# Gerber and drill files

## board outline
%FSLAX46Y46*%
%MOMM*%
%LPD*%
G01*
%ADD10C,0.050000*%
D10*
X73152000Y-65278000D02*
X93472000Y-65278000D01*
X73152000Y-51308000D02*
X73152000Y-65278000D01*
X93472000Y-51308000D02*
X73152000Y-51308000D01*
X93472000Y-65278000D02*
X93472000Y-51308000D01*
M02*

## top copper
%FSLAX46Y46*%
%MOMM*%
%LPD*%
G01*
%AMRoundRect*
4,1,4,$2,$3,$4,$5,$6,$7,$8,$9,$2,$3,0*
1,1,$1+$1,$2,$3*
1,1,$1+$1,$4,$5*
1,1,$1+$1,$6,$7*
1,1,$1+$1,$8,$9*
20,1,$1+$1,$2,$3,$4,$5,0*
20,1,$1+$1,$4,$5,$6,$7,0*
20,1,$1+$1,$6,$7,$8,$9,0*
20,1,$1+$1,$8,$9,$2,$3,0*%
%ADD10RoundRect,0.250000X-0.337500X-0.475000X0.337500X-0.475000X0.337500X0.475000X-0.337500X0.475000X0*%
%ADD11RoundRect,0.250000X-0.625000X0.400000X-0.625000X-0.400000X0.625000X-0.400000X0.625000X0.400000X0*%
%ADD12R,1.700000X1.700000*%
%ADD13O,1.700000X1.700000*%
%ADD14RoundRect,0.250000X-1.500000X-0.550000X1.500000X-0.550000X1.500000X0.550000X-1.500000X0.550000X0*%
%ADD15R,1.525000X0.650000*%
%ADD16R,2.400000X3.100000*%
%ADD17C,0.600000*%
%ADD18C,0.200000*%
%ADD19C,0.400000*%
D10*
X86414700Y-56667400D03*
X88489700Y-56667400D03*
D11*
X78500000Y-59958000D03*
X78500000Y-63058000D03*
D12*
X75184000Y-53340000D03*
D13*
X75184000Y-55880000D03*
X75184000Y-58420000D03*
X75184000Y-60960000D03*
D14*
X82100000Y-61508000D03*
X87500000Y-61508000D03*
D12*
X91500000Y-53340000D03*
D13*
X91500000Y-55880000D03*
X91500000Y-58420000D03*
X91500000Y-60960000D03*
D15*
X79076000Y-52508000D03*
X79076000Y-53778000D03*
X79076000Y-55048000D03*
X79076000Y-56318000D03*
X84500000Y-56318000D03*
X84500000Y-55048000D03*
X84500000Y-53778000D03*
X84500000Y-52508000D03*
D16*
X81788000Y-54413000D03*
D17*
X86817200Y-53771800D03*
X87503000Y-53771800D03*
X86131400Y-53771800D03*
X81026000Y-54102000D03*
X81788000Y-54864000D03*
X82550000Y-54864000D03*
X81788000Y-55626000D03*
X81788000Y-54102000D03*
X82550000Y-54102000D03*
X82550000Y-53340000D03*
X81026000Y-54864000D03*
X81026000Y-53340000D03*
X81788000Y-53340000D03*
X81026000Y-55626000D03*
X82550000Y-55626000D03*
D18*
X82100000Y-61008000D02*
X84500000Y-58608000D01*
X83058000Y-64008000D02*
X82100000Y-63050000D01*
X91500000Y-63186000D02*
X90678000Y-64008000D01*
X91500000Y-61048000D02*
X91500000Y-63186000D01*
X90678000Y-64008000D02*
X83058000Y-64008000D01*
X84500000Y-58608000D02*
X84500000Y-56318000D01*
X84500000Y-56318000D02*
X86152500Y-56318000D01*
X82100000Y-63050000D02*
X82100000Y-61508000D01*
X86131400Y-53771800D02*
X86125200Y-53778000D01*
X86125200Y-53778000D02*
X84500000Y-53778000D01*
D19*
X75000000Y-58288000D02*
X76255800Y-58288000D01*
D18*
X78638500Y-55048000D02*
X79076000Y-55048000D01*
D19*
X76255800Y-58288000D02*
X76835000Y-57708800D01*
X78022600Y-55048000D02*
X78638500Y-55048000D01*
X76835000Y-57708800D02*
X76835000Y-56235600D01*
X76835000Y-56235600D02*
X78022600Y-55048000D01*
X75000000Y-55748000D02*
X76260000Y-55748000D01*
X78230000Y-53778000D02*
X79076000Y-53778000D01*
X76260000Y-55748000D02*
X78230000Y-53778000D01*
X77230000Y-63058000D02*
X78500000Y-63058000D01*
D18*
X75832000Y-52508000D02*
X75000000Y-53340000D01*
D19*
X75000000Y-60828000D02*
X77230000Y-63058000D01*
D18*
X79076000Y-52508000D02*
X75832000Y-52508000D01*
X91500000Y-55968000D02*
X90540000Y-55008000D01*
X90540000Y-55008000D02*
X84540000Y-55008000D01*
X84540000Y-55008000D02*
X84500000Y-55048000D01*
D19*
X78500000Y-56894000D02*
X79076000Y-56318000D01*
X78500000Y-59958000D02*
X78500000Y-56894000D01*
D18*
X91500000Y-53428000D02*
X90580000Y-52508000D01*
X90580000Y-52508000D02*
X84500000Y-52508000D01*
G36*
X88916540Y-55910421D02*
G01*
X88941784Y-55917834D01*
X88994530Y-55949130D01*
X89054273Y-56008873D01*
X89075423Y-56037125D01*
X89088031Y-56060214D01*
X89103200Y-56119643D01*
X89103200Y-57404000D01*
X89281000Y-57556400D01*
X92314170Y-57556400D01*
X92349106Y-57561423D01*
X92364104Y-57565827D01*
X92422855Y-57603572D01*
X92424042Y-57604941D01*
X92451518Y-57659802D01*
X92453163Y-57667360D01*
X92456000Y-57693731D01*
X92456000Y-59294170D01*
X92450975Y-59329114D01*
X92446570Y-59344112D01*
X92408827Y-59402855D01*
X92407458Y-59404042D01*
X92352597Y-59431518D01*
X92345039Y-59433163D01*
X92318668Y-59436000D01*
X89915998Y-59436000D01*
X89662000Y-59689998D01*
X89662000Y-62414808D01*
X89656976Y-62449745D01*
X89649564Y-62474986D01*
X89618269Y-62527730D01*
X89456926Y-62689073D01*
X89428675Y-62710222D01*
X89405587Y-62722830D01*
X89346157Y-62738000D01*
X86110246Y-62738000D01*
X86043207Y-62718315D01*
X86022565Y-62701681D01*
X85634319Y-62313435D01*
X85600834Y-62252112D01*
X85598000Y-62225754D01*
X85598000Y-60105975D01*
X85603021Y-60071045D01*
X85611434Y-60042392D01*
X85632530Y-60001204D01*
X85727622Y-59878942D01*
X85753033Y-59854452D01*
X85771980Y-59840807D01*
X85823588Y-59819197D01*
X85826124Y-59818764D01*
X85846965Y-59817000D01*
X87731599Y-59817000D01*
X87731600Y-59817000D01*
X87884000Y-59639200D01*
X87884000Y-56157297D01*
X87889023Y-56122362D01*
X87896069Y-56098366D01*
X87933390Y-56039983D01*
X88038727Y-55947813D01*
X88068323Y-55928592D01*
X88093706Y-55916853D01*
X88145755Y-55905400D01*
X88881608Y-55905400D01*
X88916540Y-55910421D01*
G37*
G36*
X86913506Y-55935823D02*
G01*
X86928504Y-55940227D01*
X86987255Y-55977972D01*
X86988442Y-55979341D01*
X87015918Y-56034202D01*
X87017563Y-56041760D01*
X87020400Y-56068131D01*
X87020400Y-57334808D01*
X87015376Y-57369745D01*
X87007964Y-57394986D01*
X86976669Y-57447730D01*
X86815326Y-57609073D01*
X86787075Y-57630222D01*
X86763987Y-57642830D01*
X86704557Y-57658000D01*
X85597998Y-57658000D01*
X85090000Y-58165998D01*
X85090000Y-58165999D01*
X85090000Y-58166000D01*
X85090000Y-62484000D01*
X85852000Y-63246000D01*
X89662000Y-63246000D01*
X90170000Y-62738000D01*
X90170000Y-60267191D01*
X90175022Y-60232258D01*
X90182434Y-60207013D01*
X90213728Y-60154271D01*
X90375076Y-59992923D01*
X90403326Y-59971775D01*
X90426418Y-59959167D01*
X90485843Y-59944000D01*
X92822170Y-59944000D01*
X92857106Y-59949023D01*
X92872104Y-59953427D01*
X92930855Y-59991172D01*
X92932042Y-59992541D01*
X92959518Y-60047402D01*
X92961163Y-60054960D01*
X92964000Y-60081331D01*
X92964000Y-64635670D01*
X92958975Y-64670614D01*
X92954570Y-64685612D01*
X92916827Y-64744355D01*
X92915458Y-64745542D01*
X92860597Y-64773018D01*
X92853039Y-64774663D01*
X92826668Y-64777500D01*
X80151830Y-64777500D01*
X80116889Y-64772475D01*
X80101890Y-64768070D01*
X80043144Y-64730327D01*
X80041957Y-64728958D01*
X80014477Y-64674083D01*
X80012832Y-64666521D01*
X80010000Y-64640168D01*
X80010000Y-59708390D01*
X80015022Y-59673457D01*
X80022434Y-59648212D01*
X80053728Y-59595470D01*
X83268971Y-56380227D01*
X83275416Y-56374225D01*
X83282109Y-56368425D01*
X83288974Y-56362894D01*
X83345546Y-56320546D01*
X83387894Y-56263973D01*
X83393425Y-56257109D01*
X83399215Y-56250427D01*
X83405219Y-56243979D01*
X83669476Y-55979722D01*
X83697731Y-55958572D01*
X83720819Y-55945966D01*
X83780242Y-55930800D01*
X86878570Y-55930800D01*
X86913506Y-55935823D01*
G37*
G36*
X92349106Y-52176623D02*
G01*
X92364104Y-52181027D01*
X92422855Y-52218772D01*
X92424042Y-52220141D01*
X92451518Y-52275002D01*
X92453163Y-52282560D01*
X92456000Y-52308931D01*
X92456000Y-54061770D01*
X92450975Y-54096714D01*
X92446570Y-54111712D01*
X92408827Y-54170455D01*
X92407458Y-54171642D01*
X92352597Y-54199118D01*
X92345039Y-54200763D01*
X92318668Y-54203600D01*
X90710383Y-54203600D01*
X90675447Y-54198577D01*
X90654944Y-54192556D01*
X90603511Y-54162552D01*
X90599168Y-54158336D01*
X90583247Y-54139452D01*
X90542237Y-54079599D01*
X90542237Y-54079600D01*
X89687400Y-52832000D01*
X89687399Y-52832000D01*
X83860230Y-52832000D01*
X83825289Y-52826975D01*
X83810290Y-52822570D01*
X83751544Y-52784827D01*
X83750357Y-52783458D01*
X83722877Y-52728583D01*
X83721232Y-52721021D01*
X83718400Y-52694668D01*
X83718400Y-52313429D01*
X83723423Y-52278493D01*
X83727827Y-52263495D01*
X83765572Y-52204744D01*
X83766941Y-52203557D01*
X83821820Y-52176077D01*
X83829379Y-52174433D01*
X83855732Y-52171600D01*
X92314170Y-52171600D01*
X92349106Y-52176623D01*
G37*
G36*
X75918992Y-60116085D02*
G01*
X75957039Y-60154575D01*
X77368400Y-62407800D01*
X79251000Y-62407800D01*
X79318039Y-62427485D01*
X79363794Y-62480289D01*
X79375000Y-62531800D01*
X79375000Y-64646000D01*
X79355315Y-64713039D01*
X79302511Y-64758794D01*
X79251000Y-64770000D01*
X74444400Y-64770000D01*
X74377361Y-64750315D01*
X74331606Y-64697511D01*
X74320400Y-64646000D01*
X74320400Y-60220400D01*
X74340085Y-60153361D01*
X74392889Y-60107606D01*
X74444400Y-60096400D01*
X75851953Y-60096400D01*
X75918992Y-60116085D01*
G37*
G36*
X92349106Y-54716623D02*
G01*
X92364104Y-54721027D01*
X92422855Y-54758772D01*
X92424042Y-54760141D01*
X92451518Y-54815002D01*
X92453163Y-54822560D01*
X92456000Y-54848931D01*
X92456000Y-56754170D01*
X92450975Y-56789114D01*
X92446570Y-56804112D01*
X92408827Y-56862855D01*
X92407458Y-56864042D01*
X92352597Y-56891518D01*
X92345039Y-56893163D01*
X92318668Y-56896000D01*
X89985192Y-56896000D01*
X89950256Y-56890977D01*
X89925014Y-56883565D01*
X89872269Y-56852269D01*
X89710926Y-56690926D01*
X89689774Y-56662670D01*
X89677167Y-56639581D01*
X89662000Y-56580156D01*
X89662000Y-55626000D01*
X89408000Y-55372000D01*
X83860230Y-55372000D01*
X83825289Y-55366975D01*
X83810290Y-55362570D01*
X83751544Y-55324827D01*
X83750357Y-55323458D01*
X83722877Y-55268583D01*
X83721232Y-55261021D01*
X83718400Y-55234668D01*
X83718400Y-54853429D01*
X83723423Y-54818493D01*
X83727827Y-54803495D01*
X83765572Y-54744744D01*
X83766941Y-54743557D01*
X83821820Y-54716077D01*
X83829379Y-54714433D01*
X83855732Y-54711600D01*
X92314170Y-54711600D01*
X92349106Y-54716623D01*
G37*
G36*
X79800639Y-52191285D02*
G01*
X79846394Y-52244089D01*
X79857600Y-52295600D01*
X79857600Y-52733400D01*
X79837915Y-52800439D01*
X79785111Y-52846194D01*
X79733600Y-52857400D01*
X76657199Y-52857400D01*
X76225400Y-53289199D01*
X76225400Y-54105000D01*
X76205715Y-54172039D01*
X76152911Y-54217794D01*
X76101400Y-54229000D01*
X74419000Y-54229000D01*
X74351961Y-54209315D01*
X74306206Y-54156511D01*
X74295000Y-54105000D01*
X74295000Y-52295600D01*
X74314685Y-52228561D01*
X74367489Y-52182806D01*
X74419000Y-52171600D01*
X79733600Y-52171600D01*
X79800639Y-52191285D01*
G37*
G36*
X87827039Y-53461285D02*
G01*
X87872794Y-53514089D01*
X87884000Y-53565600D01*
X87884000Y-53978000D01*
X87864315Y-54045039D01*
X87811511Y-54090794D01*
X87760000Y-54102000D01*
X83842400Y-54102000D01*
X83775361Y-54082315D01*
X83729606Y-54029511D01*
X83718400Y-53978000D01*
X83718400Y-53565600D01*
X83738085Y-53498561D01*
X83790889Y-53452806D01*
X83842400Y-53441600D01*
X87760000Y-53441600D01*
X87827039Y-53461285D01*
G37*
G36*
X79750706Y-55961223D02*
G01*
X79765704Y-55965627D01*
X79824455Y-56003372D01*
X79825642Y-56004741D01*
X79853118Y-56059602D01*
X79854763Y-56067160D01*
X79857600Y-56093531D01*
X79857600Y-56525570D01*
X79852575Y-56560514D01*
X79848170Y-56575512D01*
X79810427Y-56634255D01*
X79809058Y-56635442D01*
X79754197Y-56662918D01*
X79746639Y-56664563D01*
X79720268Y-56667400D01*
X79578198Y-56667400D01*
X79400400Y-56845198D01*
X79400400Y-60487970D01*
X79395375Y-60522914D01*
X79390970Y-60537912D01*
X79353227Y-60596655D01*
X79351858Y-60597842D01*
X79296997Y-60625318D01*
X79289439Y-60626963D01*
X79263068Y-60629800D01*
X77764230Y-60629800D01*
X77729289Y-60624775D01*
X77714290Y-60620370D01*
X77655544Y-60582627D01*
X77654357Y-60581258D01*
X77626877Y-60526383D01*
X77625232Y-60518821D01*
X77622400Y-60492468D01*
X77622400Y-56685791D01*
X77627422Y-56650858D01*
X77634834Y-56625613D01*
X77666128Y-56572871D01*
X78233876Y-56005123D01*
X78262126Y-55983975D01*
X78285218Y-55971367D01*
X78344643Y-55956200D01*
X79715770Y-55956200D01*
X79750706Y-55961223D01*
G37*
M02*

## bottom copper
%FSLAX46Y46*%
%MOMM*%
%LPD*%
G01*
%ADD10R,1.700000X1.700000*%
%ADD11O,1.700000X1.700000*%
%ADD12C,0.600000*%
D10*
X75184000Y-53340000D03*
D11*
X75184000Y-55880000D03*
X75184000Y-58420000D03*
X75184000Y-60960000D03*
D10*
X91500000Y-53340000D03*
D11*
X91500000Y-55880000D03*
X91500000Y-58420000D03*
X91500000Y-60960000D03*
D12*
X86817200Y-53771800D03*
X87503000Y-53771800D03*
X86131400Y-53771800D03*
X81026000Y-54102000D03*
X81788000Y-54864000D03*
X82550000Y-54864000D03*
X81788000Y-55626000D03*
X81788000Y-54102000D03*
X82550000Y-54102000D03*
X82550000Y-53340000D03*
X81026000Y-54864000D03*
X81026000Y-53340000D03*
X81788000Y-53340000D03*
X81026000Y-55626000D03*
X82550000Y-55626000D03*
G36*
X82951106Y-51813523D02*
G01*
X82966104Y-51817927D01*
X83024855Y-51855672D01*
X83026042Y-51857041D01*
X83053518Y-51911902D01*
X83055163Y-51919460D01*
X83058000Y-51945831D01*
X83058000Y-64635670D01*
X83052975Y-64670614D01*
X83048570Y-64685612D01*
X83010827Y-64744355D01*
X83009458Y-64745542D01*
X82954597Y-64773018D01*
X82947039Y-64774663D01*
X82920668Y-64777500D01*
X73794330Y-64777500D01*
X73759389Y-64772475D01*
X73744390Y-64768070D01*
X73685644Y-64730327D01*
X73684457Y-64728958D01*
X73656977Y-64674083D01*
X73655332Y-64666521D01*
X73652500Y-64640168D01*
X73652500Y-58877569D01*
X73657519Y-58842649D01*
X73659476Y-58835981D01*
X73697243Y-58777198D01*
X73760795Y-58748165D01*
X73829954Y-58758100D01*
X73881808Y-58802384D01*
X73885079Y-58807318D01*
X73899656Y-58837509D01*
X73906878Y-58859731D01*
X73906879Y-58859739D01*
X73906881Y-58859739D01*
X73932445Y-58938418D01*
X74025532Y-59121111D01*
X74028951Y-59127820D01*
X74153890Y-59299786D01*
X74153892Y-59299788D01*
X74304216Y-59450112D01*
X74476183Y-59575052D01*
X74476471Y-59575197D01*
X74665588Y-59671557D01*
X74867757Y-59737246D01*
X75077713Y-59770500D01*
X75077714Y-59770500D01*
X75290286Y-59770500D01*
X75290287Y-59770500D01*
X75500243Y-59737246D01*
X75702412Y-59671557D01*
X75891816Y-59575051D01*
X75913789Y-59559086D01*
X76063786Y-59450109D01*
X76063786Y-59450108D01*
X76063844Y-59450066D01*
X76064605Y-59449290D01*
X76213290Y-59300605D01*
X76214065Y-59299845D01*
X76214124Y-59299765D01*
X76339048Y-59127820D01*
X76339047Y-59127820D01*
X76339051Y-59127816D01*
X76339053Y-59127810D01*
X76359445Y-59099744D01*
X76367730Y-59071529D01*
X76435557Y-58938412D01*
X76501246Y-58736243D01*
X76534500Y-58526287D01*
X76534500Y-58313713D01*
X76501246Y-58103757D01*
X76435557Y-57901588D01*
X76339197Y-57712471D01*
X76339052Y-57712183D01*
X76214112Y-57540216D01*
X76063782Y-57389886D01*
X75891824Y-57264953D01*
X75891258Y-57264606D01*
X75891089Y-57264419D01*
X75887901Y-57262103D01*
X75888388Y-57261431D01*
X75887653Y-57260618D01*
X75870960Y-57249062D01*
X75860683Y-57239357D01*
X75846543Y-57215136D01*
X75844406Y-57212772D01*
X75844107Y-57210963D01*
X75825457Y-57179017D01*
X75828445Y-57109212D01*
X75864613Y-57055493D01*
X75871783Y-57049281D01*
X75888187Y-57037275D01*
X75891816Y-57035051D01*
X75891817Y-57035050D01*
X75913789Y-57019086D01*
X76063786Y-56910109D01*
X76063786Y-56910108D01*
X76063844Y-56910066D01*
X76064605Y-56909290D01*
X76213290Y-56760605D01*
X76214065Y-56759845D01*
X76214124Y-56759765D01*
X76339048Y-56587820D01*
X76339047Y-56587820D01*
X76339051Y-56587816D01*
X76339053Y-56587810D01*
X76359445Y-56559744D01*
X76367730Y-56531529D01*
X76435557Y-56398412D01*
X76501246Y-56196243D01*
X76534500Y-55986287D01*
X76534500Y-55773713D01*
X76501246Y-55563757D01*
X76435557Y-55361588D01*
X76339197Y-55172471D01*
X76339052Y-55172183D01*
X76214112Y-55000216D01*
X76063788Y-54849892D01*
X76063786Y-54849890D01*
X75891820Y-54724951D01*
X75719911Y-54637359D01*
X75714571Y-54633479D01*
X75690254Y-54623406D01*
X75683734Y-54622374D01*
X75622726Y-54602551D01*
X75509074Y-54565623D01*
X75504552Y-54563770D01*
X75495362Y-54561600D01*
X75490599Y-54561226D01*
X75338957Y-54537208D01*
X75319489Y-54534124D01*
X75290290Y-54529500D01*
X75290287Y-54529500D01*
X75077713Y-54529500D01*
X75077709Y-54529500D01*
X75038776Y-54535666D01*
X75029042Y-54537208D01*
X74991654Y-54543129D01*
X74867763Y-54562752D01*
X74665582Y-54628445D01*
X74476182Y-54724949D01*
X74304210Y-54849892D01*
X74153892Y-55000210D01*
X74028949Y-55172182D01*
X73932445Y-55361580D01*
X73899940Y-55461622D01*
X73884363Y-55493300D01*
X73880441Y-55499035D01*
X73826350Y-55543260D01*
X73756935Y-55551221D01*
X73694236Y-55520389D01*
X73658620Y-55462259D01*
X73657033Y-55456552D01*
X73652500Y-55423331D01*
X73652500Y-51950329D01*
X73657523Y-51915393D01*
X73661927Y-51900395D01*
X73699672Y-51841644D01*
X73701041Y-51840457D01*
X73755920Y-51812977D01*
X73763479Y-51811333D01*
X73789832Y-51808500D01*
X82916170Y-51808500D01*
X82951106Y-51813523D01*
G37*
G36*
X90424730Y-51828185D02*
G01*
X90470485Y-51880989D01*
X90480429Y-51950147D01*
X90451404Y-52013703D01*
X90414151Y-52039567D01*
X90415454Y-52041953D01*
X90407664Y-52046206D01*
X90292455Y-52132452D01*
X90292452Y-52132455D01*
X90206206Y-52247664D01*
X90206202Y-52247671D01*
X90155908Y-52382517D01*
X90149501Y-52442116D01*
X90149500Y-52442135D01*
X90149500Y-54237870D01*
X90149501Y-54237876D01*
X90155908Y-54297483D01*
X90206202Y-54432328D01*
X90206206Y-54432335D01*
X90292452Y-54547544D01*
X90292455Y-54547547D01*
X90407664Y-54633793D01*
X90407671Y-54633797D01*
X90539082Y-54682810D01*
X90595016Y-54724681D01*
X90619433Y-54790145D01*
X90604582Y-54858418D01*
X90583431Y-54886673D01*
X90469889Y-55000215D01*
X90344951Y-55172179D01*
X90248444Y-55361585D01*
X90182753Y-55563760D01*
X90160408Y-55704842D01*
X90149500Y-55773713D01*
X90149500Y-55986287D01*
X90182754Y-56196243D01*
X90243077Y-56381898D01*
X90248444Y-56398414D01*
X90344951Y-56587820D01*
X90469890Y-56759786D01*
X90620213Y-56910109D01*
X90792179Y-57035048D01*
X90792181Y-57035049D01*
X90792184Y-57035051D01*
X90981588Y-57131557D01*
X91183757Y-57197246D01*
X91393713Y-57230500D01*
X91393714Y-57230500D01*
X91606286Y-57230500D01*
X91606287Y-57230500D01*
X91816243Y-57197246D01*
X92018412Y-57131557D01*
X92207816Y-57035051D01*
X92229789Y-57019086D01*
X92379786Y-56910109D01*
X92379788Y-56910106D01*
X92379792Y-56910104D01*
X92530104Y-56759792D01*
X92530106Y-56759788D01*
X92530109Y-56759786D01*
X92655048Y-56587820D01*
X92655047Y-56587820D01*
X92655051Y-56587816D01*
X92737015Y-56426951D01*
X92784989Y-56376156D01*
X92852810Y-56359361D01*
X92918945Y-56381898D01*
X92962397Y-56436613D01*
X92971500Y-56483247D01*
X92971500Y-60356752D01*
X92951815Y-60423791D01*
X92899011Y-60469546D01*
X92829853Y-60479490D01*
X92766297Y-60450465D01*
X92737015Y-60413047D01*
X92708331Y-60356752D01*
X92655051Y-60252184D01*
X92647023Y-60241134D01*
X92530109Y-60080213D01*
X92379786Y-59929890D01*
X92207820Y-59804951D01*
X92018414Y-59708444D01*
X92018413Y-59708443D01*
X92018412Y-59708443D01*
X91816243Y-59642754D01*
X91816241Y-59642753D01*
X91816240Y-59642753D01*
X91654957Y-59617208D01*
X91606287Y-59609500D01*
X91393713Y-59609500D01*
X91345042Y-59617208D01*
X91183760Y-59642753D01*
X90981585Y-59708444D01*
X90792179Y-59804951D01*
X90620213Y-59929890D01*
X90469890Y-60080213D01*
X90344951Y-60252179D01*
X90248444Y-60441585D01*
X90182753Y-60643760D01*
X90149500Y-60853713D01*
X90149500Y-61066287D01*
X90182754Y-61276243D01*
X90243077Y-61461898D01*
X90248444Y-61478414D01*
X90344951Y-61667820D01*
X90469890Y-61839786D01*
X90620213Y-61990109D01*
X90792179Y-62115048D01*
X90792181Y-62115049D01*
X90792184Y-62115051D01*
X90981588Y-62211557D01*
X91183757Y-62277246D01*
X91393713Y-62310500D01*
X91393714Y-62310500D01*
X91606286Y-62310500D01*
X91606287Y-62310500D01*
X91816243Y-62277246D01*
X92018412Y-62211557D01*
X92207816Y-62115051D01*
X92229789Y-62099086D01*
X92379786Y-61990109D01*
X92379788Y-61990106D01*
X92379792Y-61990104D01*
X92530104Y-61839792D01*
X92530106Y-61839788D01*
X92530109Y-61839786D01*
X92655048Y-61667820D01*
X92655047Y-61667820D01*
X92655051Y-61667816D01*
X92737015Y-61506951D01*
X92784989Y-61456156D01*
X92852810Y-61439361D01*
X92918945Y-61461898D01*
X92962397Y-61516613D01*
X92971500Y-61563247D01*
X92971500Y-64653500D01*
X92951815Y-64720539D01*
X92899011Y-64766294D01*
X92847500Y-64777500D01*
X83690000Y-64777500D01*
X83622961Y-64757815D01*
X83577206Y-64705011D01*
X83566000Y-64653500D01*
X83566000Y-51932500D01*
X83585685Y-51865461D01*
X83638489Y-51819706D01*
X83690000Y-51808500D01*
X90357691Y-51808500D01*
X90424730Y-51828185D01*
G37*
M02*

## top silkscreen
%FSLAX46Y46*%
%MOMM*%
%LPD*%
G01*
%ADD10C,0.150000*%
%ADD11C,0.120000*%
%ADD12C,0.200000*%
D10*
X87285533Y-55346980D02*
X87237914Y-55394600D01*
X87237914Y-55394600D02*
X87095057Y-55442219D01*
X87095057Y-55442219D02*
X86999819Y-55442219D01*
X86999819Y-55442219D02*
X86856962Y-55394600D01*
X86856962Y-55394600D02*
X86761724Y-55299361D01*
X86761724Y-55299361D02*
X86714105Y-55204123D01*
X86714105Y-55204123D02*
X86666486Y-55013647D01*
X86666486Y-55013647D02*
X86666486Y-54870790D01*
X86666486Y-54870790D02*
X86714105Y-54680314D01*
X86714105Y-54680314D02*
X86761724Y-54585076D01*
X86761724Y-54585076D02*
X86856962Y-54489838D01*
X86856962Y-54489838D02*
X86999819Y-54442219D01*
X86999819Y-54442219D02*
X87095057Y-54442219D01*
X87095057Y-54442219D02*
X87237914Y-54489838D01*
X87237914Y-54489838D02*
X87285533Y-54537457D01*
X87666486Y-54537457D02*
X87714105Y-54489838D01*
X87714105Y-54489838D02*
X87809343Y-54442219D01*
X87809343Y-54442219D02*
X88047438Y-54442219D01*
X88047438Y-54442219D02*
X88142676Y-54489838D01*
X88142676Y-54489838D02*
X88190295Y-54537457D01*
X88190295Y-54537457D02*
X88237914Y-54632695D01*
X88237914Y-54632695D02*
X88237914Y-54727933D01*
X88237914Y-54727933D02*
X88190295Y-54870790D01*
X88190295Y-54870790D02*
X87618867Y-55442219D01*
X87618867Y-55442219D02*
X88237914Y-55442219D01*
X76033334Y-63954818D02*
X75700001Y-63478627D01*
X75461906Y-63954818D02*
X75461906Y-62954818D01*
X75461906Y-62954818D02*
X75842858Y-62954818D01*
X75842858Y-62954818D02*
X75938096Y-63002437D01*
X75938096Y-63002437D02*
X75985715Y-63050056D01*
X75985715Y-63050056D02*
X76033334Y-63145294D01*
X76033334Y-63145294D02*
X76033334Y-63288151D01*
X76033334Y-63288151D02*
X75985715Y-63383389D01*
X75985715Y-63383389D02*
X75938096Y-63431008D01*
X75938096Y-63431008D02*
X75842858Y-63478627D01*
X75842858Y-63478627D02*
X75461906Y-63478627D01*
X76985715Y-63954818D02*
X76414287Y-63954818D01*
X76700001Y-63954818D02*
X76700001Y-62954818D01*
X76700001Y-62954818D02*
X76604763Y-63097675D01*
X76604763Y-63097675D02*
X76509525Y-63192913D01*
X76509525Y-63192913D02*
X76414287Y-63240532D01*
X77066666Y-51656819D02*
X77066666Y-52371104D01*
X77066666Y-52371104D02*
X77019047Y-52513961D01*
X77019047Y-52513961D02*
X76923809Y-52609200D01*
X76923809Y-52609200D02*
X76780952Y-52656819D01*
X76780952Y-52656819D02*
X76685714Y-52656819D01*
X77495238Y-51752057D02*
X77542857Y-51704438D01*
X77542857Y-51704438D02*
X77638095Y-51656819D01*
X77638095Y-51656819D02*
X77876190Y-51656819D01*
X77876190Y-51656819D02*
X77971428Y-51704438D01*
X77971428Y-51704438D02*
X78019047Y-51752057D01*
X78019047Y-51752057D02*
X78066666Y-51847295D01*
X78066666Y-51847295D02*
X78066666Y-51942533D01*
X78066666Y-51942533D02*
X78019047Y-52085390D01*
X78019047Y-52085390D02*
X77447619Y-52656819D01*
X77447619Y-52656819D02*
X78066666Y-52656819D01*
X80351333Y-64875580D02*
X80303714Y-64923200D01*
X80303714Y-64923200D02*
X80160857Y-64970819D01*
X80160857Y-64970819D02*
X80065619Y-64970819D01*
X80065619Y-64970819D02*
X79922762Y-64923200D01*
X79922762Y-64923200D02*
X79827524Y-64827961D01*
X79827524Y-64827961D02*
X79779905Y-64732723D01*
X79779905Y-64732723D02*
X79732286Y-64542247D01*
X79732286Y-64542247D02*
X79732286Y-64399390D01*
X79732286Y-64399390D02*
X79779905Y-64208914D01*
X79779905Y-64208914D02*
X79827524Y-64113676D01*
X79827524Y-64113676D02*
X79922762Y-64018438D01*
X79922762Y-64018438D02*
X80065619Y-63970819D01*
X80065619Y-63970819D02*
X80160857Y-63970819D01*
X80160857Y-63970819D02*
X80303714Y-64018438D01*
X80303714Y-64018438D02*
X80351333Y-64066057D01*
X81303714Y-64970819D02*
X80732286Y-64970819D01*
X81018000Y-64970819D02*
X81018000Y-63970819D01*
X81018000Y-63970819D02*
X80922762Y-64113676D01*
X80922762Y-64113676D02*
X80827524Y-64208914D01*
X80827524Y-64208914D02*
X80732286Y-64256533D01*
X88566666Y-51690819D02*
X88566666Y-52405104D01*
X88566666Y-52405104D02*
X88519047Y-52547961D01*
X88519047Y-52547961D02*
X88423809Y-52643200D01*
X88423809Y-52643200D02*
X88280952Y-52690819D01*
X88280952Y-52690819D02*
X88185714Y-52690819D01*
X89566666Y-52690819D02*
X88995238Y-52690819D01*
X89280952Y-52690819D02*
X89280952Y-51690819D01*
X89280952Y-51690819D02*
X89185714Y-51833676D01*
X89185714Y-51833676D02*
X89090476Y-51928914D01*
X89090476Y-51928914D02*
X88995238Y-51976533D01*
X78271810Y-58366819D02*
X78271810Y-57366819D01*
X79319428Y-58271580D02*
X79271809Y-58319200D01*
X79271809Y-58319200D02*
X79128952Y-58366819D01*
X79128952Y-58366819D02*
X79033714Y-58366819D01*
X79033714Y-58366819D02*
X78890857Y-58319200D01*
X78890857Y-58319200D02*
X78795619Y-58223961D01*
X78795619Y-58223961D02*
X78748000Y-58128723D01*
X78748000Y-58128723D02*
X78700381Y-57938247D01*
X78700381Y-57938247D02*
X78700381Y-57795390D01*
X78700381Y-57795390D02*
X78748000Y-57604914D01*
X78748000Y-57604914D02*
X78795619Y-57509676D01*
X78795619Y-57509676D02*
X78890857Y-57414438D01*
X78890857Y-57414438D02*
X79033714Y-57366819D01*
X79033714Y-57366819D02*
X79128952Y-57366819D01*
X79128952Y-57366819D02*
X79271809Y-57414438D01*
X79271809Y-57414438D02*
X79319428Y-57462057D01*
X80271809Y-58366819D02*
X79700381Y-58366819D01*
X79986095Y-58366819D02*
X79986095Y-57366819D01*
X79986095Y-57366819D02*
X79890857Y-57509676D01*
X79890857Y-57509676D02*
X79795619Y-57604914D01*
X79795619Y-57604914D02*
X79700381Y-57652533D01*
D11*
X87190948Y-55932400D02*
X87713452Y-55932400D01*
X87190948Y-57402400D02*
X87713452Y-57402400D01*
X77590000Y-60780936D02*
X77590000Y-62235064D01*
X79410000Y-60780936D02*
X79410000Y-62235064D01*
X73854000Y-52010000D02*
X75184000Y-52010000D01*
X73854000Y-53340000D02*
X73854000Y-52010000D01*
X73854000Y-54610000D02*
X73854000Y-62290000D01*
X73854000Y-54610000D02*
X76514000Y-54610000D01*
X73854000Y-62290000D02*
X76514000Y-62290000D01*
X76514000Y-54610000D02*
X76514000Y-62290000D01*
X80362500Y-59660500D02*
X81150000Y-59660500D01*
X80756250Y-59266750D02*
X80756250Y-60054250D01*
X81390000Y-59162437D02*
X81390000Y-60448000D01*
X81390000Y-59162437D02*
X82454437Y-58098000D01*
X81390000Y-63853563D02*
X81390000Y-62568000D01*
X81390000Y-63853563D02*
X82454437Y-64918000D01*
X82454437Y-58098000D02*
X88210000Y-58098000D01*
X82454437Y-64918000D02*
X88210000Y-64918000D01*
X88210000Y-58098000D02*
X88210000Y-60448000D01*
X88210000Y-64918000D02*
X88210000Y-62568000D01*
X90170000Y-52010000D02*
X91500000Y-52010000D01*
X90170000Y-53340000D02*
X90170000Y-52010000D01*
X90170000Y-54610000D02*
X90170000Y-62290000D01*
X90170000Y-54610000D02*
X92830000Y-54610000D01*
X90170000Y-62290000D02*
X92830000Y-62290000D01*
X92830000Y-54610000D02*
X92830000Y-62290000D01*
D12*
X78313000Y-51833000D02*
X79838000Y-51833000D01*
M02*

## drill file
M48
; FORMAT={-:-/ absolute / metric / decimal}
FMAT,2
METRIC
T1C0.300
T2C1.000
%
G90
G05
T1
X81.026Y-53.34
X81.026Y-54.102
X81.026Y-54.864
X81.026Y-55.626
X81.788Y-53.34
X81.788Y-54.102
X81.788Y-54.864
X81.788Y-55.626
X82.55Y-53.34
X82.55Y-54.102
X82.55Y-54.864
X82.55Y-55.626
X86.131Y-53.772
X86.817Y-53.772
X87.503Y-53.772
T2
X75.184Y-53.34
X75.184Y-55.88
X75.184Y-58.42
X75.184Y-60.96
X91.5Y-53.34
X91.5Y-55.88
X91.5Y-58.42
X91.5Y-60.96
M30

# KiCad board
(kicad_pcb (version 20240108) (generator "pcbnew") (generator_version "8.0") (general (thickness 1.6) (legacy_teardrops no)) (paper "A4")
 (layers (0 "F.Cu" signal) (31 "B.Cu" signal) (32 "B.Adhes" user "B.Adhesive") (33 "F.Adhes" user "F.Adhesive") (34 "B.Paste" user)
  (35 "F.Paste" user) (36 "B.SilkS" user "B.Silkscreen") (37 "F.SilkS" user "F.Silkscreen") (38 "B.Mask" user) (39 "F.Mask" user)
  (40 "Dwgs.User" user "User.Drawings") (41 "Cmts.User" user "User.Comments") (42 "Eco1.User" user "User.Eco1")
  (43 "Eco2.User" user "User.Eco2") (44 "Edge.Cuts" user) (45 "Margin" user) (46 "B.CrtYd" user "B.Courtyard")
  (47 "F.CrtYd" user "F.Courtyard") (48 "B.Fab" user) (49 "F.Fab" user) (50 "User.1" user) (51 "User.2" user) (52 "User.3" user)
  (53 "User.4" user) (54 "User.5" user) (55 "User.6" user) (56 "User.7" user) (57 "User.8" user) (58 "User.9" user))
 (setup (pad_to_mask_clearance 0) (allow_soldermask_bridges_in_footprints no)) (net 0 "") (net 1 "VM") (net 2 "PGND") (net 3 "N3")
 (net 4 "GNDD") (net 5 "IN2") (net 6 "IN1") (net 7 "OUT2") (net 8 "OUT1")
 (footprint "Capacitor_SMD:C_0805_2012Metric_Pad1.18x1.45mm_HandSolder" (layer "F.Cu") (at 87.4522 56.6674)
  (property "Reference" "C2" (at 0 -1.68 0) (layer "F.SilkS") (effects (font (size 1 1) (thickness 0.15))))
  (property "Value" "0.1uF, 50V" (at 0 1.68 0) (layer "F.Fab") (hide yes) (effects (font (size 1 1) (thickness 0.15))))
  (fp_line (start -0.261252 -0.735) (end 0.261252 -0.735) (stroke (width 0.12) (type solid)) (layer "F.SilkS"))
  (fp_line (start -0.261252 0.735) (end 0.261252 0.735) (stroke (width 0.12) (type solid)) (layer "F.SilkS"))
  (pad "1" smd roundrect (at -1.0375 0) (size 1.175 1.45) (layers "F.Cu" "F.Paste" "F.Mask") (roundrect_rratio 0.212766) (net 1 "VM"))
  (pad "2" smd roundrect (at 1.0375 0) (size 1.175 1.45) (layers "F.Cu" "F.Paste" "F.Mask") (roundrect_rratio 0.212766) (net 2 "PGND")))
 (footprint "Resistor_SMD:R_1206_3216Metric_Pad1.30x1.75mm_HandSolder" (layer "F.Cu") (at 78.5 61.508 -90)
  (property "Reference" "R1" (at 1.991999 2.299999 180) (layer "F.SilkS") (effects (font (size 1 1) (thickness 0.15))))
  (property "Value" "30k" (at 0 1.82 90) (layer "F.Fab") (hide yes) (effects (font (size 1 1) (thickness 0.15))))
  (fp_line (start -0.727064 0.91) (end 0.727064 0.91) (stroke (width 0.12) (type solid)) (layer "F.SilkS"))
  (fp_line (start -0.727064 -0.91) (end 0.727064 -0.91) (stroke (width 0.12) (type solid)) (layer "F.SilkS"))
  (pad "1" smd roundrect (at -1.55 0 270) (size 1.3 1.75) (layers "F.Cu" "F.Paste" "F.Mask") (roundrect_rratio 0.192308) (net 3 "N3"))
  (pad "2" smd roundrect (at 1.55 0 270) (size 1.3 1.75) (layers "F.Cu" "F.Paste" "F.Mask") (roundrect_rratio 0.192308) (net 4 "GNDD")))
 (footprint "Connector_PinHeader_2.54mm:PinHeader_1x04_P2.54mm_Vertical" (layer "F.Cu") (at 75.184 53.34)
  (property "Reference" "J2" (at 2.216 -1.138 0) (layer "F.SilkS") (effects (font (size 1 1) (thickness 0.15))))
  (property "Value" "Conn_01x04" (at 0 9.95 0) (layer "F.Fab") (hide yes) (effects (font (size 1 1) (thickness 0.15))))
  (fp_line (start -1.33 -1.33) (end 0 -1.33) (stroke (width 0.12) (type solid)) (layer "F.SilkS"))
  (fp_line (start -1.33 0) (end -1.33 -1.33) (stroke (width 0.12) (type solid)) (layer "F.SilkS"))
  (fp_line (start -1.33 1.27) (end -1.33 8.95) (stroke (width 0.12) (type solid)) (layer "F.SilkS"))
  (fp_line (start -1.33 1.27) (end 1.33 1.27) (stroke (width 0.12) (type solid)) (layer "F.SilkS"))
  (fp_line (start -1.33 8.95) (end 1.33 8.95) (stroke (width 0.12) (type solid)) (layer "F.SilkS"))
  (fp_line (start 1.33 1.27) (end 1.33 8.95) (stroke (width 0.12) (type solid)) (layer "F.SilkS"))
  (pad "1" thru_hole rect (at 0 0) (size 1.7 1.7) (drill 1) (layers "*.Cu" "*.Mask") (remove_unused_layers no) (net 4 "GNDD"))
  (pad "2" thru_hole oval (at 0 2.54) (size 1.7 1.7) (drill 1) (layers "*.Cu" "*.Mask") (remove_unused_layers no) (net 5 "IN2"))
  (pad "3" thru_hole oval (at 0 5.08) (size 1.7 1.7) (drill 1) (layers "*.Cu" "*.Mask") (remove_unused_layers no) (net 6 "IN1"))
  (pad "4" thru_hole oval (at 0 7.62) (size 1.7 1.7) (drill 1) (layers "*.Cu" "*.Mask") (remove_unused_layers no) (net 4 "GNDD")))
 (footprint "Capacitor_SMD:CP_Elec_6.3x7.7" (layer "F.Cu") (at 84.8 61.508)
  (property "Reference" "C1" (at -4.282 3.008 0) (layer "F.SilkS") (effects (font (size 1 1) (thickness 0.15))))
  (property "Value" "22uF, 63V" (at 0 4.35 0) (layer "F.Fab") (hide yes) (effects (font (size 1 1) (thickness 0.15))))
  (fp_line (start -4.4375 -1.8475) (end -3.65 -1.8475) (stroke (width 0.12) (type solid)) (layer "F.SilkS"))
  (fp_line (start -4.04375 -2.24125) (end -4.04375 -1.45375) (stroke (width 0.12) (type solid)) (layer "F.SilkS"))
  (fp_line (start -3.41 -2.345563) (end -3.41 -1.06) (stroke (width 0.12) (type solid)) (layer "F.SilkS"))
  (fp_line (start -3.41 -2.345563) (end -2.345563 -3.41) (stroke (width 0.12) (type solid)) (layer "F.SilkS"))
  (fp_line (start -3.41 2.345563) (end -3.41 1.06) (stroke (width 0.12) (type solid)) (layer "F.SilkS"))
  (fp_line (start -3.41 2.345563) (end -2.345563 3.41) (stroke (width 0.12) (type solid)) (layer "F.SilkS"))
  (fp_line (start -2.345563 -3.41) (end 3.41 -3.41) (stroke (width 0.12) (type solid)) (layer "F.SilkS"))
  (fp_line (start -2.345563 3.41) (end 3.41 3.41) (stroke (width 0.12) (type solid)) (layer "F.SilkS"))
  (fp_line (start 3.41 -3.41) (end 3.41 -1.06) (stroke (width 0.12) (type solid)) (layer "F.SilkS"))
  (fp_line (start 3.41 3.41) (end 3.41 1.06) (stroke (width 0.12) (type solid)) (layer "F.SilkS"))
  (pad "1" smd roundrect (at -2.7 0) (size 3.5 1.6) (layers "F.Cu" "F.Paste" "F.Mask") (roundrect_rratio 0.15625) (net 1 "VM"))
  (pad "2" smd roundrect (at 2.7 0) (size 3.5 1.6) (layers "F.Cu" "F.Paste" "F.Mask") (roundrect_rratio 0.15625) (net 2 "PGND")))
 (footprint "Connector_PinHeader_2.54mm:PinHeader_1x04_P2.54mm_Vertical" (layer "F.Cu") (at 91.5 53.34)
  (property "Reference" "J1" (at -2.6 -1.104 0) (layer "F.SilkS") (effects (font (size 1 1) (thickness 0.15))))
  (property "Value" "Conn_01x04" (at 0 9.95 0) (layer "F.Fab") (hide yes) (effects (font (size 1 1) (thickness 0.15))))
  (fp_line (start -1.33 -1.33) (end 0 -1.33) (stroke (width 0.12) (type solid)) (layer "F.SilkS"))
  (fp_line (start -1.33 0) (end -1.33 -1.33) (stroke (width 0.12) (type solid)) (layer "F.SilkS"))
  (fp_line (start -1.33 1.27) (end -1.33 8.95) (stroke (width 0.12) (type solid)) (layer "F.SilkS"))
  (fp_line (start -1.33 1.27) (end 1.33 1.27) (stroke (width 0.12) (type solid)) (layer "F.SilkS"))
  (fp_line (start -1.33 8.95) (end 1.33 8.95) (stroke (width 0.12) (type solid)) (layer "F.SilkS"))
  (fp_line (start 1.33 1.27) (end 1.33 8.95) (stroke (width 0.12) (type solid)) (layer "F.SilkS"))
  (pad "1" thru_hole rect (at 0 0) (size 1.7 1.7) (drill 1) (layers "*.Cu" "*.Mask") (remove_unused_layers no) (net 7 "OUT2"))
  (pad "2" thru_hole oval (at 0 2.54) (size 1.7 1.7) (drill 1) (layers "*.Cu" "*.Mask") (remove_unused_layers no) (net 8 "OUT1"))
  (pad "3" thru_hole oval (at 0 5.08) (size 1.7 1.7) (drill 1) (layers "*.Cu" "*.Mask") (remove_unused_layers no) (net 2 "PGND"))
  (pad "4" thru_hole oval (at 0 7.62) (size 1.7 1.7) (drill 1) (layers "*.Cu" "*.Mask") (remove_unused_layers no) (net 1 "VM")))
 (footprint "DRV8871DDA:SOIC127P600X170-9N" (layer "F.Cu") (at 81.788 54.413)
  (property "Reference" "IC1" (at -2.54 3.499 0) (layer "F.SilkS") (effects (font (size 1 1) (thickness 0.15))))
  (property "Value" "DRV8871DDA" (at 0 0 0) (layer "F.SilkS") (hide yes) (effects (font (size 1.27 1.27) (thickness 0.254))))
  (fp_line (start -3.475 -2.58) (end -1.95 -2.58) (stroke (width 0.2) (type solid)) (layer "F.SilkS"))
  (pad "1" smd rect (at -2.712 -1.905 90) (size 0.65 1.525) (layers "F.Cu" "F.Paste" "F.Mask") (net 4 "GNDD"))
  (pad "2" smd rect (at -2.712 -0.635 90) (size 0.65 1.525) (layers "F.Cu" "F.Paste" "F.Mask") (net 5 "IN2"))
  (pad "3" smd rect (at -2.712 0.635 90) (size 0.65 1.525) (layers "F.Cu" "F.Paste" "F.Mask") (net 6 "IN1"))
  (pad "4" smd rect (at -2.712 1.905 90) (size 0.65 1.525) (layers "F.Cu" "F.Paste" "F.Mask") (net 3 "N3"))
  (pad "5" smd rect (at 2.712 1.905 90) (size 0.65 1.525) (layers "F.Cu" "F.Paste" "F.Mask") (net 1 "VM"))
  (pad "6" smd rect (at 2.712 0.635 90) (size 0.65 1.525) (layers "F.Cu" "F.Paste" "F.Mask") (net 8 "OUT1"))
  (pad "7" smd rect (at 2.712 -0.635 90) (size 0.65 1.525) (layers "F.Cu" "F.Paste" "F.Mask") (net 2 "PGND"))
  (pad "8" smd rect (at 2.712 -1.905 90) (size 0.65 1.525) (layers "F.Cu" "F.Paste" "F.Mask") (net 7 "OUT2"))
  (pad "9" smd rect (at 0 0) (size 2.4 3.1) (layers "F.Cu" "F.Paste" "F.Mask") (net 4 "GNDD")))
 (gr_line (start 73.152 65.278) (end 93.472 65.278) (stroke (width 0.05) (type default)) (layer "Edge.Cuts"))
 (gr_line (start 73.152 51.308) (end 73.152 65.278) (stroke (width 0.05) (type default)) (layer "Edge.Cuts"))
 (gr_line (start 93.472 51.308) (end 73.152 51.308) (stroke (width 0.05) (type default)) (layer "Edge.Cuts"))
 (gr_line (start 93.472 65.278) (end 93.472 51.308) (stroke (width 0.05) (type default)) (layer "Edge.Cuts"))
 (segment (start 82.1 61.008) (end 84.5 58.608) (width 0.2) (layer "F.Cu") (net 1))
 (segment (start 83.058 64.008) (end 82.1 63.05) (width 0.2) (layer "F.Cu") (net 1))
 (segment (start 91.5 63.186) (end 90.678 64.008) (width 0.2) (layer "F.Cu") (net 1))
 (segment (start 91.5 61.048) (end 91.5 63.186) (width 0.2) (layer "F.Cu") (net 1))
 (segment (start 90.678 64.008) (end 83.058 64.008) (width 0.2) (layer "F.Cu") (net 1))
 (segment (start 84.5 58.608) (end 84.5 56.318) (width 0.2) (layer "F.Cu") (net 1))
 (segment (start 84.5 56.318) (end 86.1525 56.318) (width 0.2) (layer "F.Cu") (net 1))
 (segment (start 82.1 63.05) (end 82.1 61.508) (width 0.2) (layer "F.Cu") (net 1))
 (segment (start 86.1314 53.7718) (end 86.1252 53.778) (width 0.2) (layer "F.Cu") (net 2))
 (segment (start 86.1252 53.778) (end 84.5 53.778) (width 0.2) (layer "F.Cu") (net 2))
 (via (at 86.8172 53.7718) (size 0.6) (drill 0.3) (layers "F.Cu" "B.Cu") (free yes) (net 2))
 (via (at 87.503 53.7718) (size 0.6) (drill 0.3) (layers "F.Cu" "B.Cu") (free yes) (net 2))
 (via (at 86.1314 53.7718) (size 0.6) (drill 0.3) (layers "F.Cu" "B.Cu") (free yes) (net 2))
 (segment (start 75 58.288) (end 76.2558 58.288) (width 0.4) (layer "F.Cu") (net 6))
 (segment (start 78.6385 55.048) (end 79.076 55.048) (width 0.2) (layer "F.Cu") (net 6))
 (segment (start 76.2558 58.288) (end 76.835 57.7088) (width 0.4) (layer "F.Cu") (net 6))
 (segment (start 78.0226 55.048) (end 78.6385 55.048) (width 0.4) (layer "F.Cu") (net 6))
 (segment (start 76.835 57.7088) (end 76.835 56.2356) (width 0.4) (layer "F.Cu") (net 6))
 (segment (start 76.835 56.2356) (end 78.0226 55.048) (width 0.4) (layer "F.Cu") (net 6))
 (segment (start 75 55.748) (end 76.26 55.748) (width 0.4) (layer "F.Cu") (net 5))
 (segment (start 78.23 53.778) (end 79.076 53.778) (width 0.4) (layer "F.Cu") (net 5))
 (segment (start 76.26 55.748) (end 78.23 53.778) (width 0.4) (layer "F.Cu") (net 5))
 (segment (start 77.23 63.058) (end 78.5 63.058) (width 0.4) (layer "F.Cu") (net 4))
 (segment (start 75.832 52.508) (end 75 53.34) (width 0.2) (layer "F.Cu") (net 4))
 (segment (start 75 60.828) (end 77.23 63.058) (width 0.4) (layer "F.Cu") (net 4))
 (segment (start 79.076 52.508) (end 75.832 52.508) (width 0.2) (layer "F.Cu") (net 4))
 (via (at 81.026 54.102) (size 0.6) (drill 0.3) (layers "F.Cu" "B.Cu") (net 4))
 (via (at 81.788 54.864) (size 0.6) (drill 0.3) (layers "F.Cu" "B.Cu") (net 4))
 (via (at 82.55 54.864) (size 0.6) (drill 0.3) (layers "F.Cu" "B.Cu") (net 4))
 (via (at 81.788 55.626) (size 0.6) (drill 0.3) (layers "F.Cu" "B.Cu") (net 4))
 (via (at 81.788 54.102) (size 0.6) (drill 0.3) (layers "F.Cu" "B.Cu") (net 4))
 (via (at 82.55 54.102) (size 0.6) (drill 0.3) (layers "F.Cu" "B.Cu") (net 4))
 (via (at 82.55 53.34) (size 0.6) (drill 0.3) (layers "F.Cu" "B.Cu") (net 4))
 (via (at 81.026 54.864) (size 0.6) (drill 0.3) (layers "F.Cu" "B.Cu") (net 4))
 (via (at 81.026 53.34) (size 0.6) (drill 0.3) (layers "F.Cu" "B.Cu") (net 4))
 (via (at 81.788 53.34) (size 0.6) (drill 0.3) (layers "F.Cu" "B.Cu") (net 4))
 (via (at 81.026 55.626) (size 0.6) (drill 0.3) (layers "F.Cu" "B.Cu") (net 4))
 (via (at 82.55 55.626) (size 0.6) (drill 0.3) (layers "F.Cu" "B.Cu") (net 4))
 (segment (start 91.5 55.968) (end 90.54 55.008) (width 0.2) (layer "F.Cu") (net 8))
 (segment (start 90.54 55.008) (end 84.54 55.008) (width 0.2) (layer "F.Cu") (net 8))
 (segment (start 84.54 55.008) (end 84.5 55.048) (width 0.2) (layer "F.Cu") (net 8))
 (segment (start 78.5 56.894) (end 79.076 56.318) (width 0.4) (layer "F.Cu") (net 3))
 (segment (start 78.5 59.958) (end 78.5 56.894) (width 0.4) (layer "F.Cu") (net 3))
 (segment (start 91.5 53.428) (end 90.58 52.508) (width 0.2) (layer "F.Cu") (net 7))
 (segment (start 90.58 52.508) (end 84.5 52.508) (width 0.2) (layer "F.Cu") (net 7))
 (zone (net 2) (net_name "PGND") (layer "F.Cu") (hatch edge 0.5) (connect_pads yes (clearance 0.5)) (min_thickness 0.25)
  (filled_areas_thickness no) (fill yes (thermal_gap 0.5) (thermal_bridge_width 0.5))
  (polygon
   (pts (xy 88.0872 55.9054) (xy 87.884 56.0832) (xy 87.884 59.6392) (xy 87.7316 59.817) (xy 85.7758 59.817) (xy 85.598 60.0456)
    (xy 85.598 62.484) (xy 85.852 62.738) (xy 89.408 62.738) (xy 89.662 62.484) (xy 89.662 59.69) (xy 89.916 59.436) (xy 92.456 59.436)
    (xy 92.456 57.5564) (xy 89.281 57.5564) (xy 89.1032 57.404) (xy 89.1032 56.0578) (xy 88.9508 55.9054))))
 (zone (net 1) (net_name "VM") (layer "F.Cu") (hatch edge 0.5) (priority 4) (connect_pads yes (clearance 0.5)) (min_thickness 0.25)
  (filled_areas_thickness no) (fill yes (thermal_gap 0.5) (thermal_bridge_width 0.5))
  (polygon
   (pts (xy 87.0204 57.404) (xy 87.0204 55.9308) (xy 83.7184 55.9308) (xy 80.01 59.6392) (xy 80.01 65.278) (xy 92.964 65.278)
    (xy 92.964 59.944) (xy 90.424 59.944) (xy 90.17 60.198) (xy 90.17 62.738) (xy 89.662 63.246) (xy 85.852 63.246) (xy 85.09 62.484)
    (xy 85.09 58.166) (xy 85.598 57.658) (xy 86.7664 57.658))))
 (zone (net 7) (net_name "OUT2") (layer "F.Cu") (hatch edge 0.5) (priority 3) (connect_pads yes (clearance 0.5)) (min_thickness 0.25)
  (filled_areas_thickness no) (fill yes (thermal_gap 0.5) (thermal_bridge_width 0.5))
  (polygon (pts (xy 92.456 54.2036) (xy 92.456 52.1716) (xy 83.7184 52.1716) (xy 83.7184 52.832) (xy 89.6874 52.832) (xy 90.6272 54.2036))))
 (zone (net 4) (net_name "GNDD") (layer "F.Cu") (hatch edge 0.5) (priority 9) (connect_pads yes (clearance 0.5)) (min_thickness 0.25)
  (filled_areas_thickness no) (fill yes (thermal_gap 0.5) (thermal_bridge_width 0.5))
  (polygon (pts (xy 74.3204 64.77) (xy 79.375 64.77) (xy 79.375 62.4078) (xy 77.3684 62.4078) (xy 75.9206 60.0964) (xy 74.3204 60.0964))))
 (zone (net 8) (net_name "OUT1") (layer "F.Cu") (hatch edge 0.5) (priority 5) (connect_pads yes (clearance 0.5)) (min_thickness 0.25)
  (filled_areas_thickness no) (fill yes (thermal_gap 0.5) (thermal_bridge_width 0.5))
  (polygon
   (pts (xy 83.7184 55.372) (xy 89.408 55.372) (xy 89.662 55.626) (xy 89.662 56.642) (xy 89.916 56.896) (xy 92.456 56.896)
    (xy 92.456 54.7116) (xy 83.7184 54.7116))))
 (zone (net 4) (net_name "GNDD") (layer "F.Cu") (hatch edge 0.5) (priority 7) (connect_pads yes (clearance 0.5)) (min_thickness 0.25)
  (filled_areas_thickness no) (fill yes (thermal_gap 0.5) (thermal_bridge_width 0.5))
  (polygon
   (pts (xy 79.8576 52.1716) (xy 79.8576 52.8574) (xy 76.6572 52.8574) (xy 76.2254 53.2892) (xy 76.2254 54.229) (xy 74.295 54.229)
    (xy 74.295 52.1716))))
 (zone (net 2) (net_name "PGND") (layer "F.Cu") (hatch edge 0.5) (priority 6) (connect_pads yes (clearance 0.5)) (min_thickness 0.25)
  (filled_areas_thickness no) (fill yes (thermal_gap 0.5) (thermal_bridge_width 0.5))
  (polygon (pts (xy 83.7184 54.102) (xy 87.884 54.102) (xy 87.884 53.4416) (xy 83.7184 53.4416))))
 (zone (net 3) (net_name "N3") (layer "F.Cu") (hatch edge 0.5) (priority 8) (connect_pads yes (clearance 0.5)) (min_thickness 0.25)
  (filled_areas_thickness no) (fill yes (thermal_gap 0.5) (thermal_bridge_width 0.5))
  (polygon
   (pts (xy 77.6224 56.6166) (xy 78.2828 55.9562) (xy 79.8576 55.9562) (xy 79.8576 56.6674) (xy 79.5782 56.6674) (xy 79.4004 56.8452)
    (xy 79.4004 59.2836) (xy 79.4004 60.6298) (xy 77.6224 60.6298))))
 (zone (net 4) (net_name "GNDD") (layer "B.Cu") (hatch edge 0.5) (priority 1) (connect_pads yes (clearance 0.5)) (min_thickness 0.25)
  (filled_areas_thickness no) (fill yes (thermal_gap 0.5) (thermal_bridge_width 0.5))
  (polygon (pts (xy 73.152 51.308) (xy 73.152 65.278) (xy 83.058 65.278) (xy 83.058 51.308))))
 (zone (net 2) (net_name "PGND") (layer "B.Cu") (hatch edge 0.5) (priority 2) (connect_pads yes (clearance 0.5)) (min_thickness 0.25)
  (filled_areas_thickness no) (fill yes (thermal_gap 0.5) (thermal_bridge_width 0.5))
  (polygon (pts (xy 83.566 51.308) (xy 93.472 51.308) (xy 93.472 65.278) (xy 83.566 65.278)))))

